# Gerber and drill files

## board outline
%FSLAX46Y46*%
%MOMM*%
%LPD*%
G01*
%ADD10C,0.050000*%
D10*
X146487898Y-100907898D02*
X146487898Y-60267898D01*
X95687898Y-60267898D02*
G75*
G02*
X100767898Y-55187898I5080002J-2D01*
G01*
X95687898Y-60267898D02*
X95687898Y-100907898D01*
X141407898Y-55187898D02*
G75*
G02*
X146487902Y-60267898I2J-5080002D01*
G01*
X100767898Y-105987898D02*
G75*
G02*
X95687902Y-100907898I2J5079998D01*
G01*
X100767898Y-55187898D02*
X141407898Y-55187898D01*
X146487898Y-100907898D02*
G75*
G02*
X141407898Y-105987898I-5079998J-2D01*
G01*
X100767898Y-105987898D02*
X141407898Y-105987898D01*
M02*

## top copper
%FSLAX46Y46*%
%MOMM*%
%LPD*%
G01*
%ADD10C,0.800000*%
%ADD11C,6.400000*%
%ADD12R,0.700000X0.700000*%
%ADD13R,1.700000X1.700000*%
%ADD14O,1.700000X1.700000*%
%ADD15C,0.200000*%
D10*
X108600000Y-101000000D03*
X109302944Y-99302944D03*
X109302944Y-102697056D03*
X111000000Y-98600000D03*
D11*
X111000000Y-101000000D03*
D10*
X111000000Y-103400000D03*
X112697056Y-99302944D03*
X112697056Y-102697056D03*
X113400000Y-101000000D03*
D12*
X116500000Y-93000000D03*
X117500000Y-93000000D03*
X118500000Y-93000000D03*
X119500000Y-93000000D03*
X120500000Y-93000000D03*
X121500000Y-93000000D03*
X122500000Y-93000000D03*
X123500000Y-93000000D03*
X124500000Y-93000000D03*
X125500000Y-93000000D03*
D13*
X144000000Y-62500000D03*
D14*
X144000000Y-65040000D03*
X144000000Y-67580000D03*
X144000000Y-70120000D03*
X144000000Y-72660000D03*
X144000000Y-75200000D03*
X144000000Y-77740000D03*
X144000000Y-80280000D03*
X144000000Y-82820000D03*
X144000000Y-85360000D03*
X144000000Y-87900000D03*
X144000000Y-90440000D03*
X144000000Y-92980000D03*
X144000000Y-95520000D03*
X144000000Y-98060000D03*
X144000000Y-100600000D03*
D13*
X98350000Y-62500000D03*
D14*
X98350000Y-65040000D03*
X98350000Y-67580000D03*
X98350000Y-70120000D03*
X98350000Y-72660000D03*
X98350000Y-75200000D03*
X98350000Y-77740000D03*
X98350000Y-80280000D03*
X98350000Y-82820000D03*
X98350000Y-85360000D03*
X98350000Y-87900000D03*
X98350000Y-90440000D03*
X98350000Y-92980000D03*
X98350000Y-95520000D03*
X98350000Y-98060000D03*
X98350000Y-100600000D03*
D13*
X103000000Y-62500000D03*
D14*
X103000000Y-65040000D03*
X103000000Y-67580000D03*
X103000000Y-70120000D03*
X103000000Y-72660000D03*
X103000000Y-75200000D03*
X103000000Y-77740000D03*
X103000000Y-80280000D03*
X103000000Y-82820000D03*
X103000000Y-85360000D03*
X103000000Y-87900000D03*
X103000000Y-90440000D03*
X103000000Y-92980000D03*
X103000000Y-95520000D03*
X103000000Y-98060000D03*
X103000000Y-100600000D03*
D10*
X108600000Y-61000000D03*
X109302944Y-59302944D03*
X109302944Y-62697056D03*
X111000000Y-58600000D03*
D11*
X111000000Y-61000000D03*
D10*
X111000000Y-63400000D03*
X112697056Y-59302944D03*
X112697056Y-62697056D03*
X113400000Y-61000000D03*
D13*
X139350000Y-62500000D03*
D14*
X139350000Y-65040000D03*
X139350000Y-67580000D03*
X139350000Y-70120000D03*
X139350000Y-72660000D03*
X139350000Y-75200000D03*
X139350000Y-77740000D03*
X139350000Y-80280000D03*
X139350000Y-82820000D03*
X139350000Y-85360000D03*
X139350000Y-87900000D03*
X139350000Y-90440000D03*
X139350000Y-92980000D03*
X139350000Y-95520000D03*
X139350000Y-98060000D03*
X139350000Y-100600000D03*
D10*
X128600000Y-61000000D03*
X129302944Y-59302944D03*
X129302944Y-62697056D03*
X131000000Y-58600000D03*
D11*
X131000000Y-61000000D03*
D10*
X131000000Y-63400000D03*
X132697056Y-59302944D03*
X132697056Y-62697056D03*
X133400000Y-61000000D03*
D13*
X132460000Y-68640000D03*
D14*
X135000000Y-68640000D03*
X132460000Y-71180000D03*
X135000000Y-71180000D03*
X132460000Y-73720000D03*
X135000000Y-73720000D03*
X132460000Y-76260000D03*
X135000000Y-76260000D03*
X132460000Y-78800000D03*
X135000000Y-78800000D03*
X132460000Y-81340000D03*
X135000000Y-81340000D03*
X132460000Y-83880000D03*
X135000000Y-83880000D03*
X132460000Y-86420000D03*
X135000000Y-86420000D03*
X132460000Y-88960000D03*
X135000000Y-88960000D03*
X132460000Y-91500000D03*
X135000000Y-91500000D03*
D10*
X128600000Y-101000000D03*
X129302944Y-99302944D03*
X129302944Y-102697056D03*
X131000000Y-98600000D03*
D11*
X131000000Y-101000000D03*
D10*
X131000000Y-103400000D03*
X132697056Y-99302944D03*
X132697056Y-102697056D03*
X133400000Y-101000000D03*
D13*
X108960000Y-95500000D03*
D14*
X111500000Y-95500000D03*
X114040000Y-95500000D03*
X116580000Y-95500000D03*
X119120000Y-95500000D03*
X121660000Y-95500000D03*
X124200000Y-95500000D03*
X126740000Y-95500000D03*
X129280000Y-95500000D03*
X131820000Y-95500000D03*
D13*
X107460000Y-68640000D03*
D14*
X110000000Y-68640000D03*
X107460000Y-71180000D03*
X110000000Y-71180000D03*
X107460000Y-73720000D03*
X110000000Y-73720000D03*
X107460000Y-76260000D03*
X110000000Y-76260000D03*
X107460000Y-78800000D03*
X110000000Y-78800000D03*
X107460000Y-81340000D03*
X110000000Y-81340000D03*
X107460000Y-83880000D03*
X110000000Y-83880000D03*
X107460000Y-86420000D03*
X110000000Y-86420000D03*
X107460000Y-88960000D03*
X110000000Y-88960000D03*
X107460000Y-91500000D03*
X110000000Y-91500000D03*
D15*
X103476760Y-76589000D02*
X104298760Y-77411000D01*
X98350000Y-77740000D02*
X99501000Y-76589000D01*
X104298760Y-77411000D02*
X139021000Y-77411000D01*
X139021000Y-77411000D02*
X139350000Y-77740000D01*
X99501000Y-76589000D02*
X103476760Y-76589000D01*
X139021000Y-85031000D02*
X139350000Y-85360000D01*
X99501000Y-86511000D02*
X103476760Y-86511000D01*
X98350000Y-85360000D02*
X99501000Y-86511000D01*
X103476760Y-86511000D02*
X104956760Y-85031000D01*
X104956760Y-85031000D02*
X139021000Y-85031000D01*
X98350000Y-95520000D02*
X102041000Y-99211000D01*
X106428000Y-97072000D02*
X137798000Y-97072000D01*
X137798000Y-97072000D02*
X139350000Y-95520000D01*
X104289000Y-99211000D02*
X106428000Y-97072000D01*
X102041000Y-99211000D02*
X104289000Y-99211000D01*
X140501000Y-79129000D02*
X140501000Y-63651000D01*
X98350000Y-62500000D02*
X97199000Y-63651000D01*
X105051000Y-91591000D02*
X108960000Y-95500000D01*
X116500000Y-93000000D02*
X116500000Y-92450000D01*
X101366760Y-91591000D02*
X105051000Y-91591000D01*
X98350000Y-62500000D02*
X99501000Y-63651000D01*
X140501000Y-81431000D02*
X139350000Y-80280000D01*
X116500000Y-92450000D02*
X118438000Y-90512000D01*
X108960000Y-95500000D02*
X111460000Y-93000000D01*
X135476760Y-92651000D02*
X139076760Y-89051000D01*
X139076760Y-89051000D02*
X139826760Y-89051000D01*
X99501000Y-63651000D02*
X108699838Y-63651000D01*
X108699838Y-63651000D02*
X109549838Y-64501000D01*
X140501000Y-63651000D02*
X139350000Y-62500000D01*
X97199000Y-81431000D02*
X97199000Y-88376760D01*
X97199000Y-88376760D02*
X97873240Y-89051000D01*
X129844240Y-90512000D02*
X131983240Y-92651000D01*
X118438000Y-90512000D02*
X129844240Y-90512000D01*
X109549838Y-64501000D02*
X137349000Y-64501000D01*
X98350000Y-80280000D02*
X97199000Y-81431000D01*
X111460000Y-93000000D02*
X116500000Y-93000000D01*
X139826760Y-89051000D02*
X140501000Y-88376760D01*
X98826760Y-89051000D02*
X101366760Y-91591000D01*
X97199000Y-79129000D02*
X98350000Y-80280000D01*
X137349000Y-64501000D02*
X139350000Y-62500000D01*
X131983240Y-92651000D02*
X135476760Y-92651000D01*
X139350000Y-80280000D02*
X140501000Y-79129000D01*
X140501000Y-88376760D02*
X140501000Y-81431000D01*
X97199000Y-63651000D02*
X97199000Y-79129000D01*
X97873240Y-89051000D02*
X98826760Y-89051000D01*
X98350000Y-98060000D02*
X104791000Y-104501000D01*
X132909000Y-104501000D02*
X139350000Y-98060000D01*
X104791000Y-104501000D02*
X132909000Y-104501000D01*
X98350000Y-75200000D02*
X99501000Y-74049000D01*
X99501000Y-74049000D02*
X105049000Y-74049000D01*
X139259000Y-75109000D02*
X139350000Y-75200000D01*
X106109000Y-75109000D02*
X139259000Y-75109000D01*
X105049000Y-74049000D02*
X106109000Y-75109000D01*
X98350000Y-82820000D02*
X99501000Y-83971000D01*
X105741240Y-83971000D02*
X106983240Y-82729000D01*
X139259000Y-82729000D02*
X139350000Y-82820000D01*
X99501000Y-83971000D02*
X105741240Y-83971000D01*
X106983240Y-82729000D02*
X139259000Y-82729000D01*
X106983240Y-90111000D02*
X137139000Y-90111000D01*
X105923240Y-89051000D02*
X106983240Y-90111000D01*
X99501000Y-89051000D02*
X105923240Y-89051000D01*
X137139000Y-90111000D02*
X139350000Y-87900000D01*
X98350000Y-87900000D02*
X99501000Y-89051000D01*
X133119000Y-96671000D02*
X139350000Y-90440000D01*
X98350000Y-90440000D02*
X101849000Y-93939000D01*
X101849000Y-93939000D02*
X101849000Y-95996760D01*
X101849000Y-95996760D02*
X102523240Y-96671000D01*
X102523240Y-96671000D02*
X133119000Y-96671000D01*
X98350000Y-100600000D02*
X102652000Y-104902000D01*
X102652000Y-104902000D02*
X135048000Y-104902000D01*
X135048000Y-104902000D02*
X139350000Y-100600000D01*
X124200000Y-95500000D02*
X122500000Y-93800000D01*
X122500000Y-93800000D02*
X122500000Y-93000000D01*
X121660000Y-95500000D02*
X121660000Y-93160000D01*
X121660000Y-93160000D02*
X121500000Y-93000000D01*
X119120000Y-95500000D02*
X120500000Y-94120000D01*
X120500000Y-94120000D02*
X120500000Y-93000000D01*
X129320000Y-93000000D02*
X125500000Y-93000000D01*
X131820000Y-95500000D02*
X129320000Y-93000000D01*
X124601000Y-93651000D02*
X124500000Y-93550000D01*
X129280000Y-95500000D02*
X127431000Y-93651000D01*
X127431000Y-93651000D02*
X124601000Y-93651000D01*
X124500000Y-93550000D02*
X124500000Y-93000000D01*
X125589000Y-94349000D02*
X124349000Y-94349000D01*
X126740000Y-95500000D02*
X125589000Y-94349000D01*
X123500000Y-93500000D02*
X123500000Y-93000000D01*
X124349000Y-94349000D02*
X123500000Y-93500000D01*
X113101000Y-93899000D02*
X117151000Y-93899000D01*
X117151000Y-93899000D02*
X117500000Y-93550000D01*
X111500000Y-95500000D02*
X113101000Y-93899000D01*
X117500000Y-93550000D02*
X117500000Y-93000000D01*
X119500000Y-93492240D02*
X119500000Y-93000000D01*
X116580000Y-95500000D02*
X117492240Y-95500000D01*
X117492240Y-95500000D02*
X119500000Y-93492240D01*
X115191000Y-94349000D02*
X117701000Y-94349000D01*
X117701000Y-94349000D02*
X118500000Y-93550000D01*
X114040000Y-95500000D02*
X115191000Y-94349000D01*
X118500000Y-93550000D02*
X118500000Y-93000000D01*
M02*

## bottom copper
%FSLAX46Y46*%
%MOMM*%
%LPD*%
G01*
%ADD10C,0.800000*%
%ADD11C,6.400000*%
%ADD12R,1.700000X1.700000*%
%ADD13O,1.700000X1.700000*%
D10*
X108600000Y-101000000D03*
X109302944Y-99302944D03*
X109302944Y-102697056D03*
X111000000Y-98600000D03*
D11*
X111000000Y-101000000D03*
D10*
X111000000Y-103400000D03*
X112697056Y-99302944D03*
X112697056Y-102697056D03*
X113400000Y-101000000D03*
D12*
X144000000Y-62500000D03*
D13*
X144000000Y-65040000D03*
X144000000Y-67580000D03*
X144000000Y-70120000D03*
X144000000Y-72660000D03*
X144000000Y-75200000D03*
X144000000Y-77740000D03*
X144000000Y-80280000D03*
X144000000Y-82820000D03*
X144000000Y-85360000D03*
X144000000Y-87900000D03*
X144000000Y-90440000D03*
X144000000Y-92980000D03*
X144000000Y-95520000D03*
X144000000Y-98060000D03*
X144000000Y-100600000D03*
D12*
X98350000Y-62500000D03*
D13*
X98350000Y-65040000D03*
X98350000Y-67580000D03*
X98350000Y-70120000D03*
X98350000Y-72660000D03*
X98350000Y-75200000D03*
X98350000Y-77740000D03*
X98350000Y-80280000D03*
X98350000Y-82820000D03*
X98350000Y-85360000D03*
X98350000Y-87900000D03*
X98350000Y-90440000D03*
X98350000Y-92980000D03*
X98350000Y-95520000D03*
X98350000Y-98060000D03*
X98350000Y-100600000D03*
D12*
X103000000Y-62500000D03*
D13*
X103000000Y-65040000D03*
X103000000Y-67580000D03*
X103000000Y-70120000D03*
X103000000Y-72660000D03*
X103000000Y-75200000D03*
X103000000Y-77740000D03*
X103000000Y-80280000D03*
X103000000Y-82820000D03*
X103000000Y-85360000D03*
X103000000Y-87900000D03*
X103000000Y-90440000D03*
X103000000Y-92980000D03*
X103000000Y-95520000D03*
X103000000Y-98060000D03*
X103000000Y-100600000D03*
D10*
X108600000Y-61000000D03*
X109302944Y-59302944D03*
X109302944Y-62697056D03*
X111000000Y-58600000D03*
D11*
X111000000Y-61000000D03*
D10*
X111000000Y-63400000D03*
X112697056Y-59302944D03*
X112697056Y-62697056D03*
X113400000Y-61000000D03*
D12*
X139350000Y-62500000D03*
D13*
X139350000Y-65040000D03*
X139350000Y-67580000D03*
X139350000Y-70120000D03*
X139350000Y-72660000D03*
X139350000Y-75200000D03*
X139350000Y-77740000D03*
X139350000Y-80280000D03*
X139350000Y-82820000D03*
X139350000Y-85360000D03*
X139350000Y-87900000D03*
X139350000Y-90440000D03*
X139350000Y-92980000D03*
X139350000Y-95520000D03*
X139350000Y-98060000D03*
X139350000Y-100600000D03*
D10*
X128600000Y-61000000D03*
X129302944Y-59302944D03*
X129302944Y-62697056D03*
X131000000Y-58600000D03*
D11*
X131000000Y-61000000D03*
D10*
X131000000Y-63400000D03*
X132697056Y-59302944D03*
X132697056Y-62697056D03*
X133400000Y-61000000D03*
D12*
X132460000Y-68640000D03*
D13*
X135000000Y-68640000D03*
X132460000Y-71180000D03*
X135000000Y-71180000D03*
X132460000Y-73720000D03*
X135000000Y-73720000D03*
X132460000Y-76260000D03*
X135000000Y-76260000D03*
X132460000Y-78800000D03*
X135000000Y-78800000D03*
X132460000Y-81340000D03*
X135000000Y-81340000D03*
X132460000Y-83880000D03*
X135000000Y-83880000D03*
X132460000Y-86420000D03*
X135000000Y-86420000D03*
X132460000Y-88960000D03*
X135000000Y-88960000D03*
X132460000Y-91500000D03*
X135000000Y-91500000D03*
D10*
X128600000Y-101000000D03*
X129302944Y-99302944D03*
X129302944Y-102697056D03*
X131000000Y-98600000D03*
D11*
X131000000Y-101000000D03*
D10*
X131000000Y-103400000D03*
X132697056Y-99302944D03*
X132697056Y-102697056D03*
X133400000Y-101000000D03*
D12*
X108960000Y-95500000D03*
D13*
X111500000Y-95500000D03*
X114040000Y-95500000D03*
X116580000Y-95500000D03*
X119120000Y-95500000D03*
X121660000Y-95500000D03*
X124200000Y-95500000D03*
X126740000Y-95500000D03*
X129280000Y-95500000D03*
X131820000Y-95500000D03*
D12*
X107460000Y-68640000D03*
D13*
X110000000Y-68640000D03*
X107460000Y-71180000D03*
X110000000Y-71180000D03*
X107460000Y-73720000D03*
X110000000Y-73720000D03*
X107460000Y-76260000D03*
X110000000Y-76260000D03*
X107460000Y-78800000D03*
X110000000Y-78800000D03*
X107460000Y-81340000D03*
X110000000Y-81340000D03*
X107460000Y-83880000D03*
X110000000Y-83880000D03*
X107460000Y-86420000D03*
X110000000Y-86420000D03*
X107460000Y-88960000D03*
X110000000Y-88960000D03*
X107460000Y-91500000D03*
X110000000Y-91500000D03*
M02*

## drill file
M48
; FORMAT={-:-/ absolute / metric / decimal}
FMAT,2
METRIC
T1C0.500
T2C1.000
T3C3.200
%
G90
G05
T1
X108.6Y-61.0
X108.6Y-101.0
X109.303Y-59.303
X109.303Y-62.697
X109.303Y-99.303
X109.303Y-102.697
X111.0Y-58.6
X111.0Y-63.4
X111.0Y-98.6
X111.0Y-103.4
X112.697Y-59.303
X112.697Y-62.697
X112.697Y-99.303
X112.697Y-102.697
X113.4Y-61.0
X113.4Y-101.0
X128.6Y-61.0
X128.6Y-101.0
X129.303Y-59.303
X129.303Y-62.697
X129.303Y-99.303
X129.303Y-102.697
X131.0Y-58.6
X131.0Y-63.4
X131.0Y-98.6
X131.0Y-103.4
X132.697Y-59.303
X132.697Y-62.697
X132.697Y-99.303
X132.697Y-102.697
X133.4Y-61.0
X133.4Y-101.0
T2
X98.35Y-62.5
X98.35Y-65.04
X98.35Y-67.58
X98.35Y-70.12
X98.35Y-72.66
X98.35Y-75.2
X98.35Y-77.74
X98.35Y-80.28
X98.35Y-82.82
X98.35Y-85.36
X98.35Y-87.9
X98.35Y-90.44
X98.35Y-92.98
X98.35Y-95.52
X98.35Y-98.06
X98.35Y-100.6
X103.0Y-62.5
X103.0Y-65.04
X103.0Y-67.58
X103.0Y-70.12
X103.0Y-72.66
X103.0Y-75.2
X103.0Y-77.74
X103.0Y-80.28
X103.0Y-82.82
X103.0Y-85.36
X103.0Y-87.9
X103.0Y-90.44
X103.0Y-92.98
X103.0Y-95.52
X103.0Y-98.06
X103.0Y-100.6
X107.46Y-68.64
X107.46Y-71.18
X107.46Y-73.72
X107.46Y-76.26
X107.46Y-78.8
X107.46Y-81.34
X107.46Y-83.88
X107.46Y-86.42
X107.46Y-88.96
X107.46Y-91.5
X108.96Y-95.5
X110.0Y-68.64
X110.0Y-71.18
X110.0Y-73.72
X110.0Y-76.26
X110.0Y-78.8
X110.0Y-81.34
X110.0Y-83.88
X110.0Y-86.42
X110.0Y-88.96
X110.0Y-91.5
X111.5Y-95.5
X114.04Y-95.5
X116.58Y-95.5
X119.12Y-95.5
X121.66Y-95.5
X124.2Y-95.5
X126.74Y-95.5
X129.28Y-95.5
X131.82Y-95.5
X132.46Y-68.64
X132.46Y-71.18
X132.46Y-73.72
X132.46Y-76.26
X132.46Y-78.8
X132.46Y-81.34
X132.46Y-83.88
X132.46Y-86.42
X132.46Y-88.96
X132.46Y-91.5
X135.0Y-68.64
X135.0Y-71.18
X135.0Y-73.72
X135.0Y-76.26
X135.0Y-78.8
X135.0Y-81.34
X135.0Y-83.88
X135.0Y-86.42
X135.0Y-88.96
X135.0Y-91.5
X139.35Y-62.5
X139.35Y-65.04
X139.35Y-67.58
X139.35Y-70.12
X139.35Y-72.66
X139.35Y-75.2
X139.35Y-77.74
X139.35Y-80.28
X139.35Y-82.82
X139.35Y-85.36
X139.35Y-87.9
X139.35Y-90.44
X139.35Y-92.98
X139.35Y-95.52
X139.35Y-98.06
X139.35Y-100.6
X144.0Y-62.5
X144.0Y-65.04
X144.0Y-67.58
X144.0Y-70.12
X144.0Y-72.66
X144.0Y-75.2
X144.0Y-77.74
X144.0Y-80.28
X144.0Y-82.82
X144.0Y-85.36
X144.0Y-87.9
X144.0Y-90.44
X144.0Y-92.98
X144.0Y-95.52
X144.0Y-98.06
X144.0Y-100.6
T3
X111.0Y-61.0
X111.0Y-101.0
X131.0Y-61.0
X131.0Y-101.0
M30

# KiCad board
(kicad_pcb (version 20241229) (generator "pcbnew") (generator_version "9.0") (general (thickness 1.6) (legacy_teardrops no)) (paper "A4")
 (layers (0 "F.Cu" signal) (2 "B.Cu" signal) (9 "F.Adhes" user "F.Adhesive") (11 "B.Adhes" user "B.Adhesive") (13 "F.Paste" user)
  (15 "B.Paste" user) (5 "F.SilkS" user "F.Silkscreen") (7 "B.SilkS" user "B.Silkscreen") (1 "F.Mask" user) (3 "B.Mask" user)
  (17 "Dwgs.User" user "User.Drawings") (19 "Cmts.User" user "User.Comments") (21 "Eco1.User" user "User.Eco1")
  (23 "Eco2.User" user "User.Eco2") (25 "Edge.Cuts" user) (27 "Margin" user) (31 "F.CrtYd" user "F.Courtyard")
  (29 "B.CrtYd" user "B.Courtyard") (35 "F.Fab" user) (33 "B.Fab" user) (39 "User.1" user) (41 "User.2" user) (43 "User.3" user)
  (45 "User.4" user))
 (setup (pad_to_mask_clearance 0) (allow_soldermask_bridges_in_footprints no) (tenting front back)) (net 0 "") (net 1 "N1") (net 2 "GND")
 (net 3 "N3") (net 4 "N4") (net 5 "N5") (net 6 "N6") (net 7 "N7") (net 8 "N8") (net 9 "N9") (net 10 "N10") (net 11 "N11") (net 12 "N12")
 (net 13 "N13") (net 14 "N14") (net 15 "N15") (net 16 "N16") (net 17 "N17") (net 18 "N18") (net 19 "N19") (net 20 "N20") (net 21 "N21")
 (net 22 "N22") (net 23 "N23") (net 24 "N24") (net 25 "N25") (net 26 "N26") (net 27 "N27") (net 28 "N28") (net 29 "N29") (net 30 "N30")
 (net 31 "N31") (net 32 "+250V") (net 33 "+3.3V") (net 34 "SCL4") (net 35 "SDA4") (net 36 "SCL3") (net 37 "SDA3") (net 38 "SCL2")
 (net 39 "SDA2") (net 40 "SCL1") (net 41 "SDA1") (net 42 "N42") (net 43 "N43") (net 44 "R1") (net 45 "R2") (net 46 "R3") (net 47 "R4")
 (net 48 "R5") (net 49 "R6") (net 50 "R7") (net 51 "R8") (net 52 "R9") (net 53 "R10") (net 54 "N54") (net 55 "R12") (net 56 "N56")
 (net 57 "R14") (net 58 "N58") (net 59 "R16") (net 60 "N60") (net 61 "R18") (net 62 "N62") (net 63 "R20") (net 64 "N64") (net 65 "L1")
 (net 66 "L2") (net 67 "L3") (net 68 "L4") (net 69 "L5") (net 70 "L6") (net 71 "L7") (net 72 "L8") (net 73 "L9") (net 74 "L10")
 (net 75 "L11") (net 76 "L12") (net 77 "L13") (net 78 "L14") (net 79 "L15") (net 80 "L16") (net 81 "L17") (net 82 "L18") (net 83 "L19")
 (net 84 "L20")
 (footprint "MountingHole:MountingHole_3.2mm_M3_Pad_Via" (layer "F.Cu") (at 111 101)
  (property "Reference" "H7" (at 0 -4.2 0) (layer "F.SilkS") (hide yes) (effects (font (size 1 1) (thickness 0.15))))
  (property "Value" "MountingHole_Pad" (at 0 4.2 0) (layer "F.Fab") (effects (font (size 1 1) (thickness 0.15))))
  (pad "1" thru_hole circle (at -2.4 0) (size 0.8 0.8) (drill 0.5) (layers "*.Cu" "*.Mask") (remove_unused_layers no) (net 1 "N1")
   (zone_connect 2))
  (pad "1" thru_hole circle (at -1.697056 -1.697056) (size 0.8 0.8) (drill 0.5) (layers "*.Cu" "*.Mask") (remove_unused_layers no)
   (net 1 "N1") (zone_connect 2))
  (pad "1" thru_hole circle (at -1.697056 1.697056) (size 0.8 0.8) (drill 0.5) (layers "*.Cu" "*.Mask") (remove_unused_layers no)
   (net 1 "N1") (zone_connect 2))
  (pad "1" thru_hole circle (at 0 -2.4) (size 0.8 0.8) (drill 0.5) (layers "*.Cu" "*.Mask") (remove_unused_layers no) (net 1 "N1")
   (zone_connect 2))
  (pad "1" thru_hole circle (at 0 0) (size 6.4 6.4) (drill 3.2) (layers "*.Cu" "*.Mask") (remove_unused_layers no) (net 1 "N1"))
  (pad "1" thru_hole circle (at 0 2.4) (size 0.8 0.8) (drill 0.5) (layers "*.Cu" "*.Mask") (remove_unused_layers no) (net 1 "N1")
   (zone_connect 2))
  (pad "1" thru_hole circle (at 1.697056 -1.697056) (size 0.8 0.8) (drill 0.5) (layers "*.Cu" "*.Mask") (remove_unused_layers no)
   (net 1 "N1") (zone_connect 2))
  (pad "1" thru_hole circle (at 1.697056 1.697056) (size 0.8 0.8) (drill 0.5) (layers "*.Cu" "*.Mask") (remove_unused_layers no)
   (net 1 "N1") (zone_connect 2))
  (pad "1" thru_hole circle (at 2.4 0) (size 0.8 0.8) (drill 0.5) (layers "*.Cu" "*.Mask") (remove_unused_layers no) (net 1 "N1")
   (zone_connect 2)))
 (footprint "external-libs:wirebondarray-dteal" (layer "F.Cu") (at 116.5 93)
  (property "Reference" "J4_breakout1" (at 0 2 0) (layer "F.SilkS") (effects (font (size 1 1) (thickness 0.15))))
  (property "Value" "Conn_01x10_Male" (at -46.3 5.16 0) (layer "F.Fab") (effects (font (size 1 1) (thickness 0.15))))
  (pad "1" smd rect (at 0 0) (size 0.7 0.7) (layers "F.Cu" "F.Mask" "F.Paste") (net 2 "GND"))
  (pad "2" smd rect (at 1 0) (size 0.7 0.7) (layers "F.Cu" "F.Mask" "F.Paste") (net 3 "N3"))
  (pad "3" smd rect (at 2 0) (size 0.7 0.7) (layers "F.Cu" "F.Mask" "F.Paste") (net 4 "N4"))
  (pad "4" smd rect (at 3 0) (size 0.7 0.7) (layers "F.Cu" "F.Mask" "F.Paste") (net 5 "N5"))
  (pad "5" smd rect (at 4 0) (size 0.7 0.7) (layers "F.Cu" "F.Mask" "F.Paste") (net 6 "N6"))
  (pad "6" smd rect (at 5 0) (size 0.7 0.7) (layers "F.Cu" "F.Mask" "F.Paste") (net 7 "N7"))
  (pad "7" smd rect (at 6 0) (size 0.7 0.7) (layers "F.Cu" "F.Mask" "F.Paste") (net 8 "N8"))
  (pad "8" smd rect (at 7 0) (size 0.7 0.7) (layers "F.Cu" "F.Mask" "F.Paste") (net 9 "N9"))
  (pad "9" smd rect (at 8 0) (size 0.7 0.7) (layers "F.Cu" "F.Mask" "F.Paste") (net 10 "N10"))
  (pad "10" smd rect (at 9 0) (size 0.7 0.7) (layers "F.Cu" "F.Mask" "F.Paste") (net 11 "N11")))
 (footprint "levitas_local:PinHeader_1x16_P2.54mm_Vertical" (layer "F.Cu") (at 144 62.5)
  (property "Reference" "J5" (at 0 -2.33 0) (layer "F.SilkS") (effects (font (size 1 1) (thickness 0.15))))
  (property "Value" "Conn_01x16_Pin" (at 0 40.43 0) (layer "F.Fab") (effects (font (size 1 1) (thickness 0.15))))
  (pad "1" thru_hole rect (at 0 0) (size 1.7 1.7) (drill 1) (layers "*.Cu" "*.Mask") (remove_unused_layers no) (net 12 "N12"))
  (pad "2" thru_hole oval (at 0 2.54) (size 1.7 1.7) (drill 1) (layers "*.Cu" "*.Mask") (remove_unused_layers no) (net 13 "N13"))
  (pad "3" thru_hole oval (at 0 5.08) (size 1.7 1.7) (drill 1) (layers "*.Cu" "*.Mask") (remove_unused_layers no) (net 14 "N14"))
  (pad "4" thru_hole oval (at 0 7.62) (size 1.7 1.7) (drill 1) (layers "*.Cu" "*.Mask") (remove_unused_layers no) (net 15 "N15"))
  (pad "5" thru_hole oval (at 0 10.16) (size 1.7 1.7) (drill 1) (layers "*.Cu" "*.Mask") (remove_unused_layers no) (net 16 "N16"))
  (pad "6" thru_hole oval (at 0 12.7) (size 1.7 1.7) (drill 1) (layers "*.Cu" "*.Mask") (remove_unused_layers no) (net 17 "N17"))
  (pad "7" thru_hole oval (at 0 15.24) (size 1.7 1.7) (drill 1) (layers "*.Cu" "*.Mask") (remove_unused_layers no) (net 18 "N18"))
  (pad "8" thru_hole oval (at 0 17.78) (size 1.7 1.7) (drill 1) (layers "*.Cu" "*.Mask") (remove_unused_layers no) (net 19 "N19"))
  (pad "9" thru_hole oval (at 0 20.32) (size 1.7 1.7) (drill 1) (layers "*.Cu" "*.Mask") (remove_unused_layers no) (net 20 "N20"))
  (pad "10" thru_hole oval (at 0 22.86) (size 1.7 1.7) (drill 1) (layers "*.Cu" "*.Mask") (remove_unused_layers no) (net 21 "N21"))
  (pad "11" thru_hole oval (at 0 25.4) (size 1.7 1.7) (drill 1) (layers "*.Cu" "*.Mask") (remove_unused_layers no) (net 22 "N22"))
  (pad "12" thru_hole oval (at 0 27.94) (size 1.7 1.7) (drill 1) (layers "*.Cu" "*.Mask") (remove_unused_layers no) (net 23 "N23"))
  (pad "13" thru_hole oval (at 0 30.48) (size 1.7 1.7) (drill 1) (layers "*.Cu" "*.Mask") (remove_unused_layers no) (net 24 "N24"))
  (pad "14" thru_hole oval (at 0 33.02) (size 1.7 1.7) (drill 1) (layers "*.Cu" "*.Mask") (remove_unused_layers no) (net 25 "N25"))
  (pad "15" thru_hole oval (at 0 35.56) (size 1.7 1.7) (drill 1) (layers "*.Cu" "*.Mask") (remove_unused_layers no) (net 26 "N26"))
  (pad "16" thru_hole oval (at 0 38.1) (size 1.7 1.7) (drill 1) (layers "*.Cu" "*.Mask") (remove_unused_layers no) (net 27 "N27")))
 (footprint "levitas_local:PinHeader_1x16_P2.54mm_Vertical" (layer "F.Cu") (at 98.35 62.5)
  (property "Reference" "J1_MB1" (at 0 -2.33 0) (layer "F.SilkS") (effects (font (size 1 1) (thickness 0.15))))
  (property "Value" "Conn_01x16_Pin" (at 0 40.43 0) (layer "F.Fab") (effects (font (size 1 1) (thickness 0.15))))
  (pad "1" thru_hole rect (at 0 0) (size 1.7 1.7) (drill 1) (layers "*.Cu" "*.Mask") (remove_unused_layers no) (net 2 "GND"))
  (pad "2" thru_hole oval (at 0 2.54) (size 1.7 1.7) (drill 1) (layers "*.Cu" "*.Mask") (remove_unused_layers no) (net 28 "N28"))
  (pad "3" thru_hole oval (at 0 5.08) (size 1.7 1.7) (drill 1) (layers "*.Cu" "*.Mask") (remove_unused_layers no) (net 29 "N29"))
  (pad "4" thru_hole oval (at 0 7.62) (size 1.7 1.7) (drill 1) (layers "*.Cu" "*.Mask") (remove_unused_layers no) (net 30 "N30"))
  (pad "5" thru_hole oval (at 0 10.16) (size 1.7 1.7) (drill 1) (layers "*.Cu" "*.Mask") (remove_unused_layers no) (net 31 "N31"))
  (pad "6" thru_hole oval (at 0 12.7) (size 1.7 1.7) (drill 1) (layers "*.Cu" "*.Mask") (remove_unused_layers no) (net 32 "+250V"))
  (pad "7" thru_hole oval (at 0 15.24) (size 1.7 1.7) (drill 1) (layers "*.Cu" "*.Mask") (remove_unused_layers no) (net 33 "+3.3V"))
  (pad "8" thru_hole oval (at 0 17.78) (size 1.7 1.7) (drill 1) (layers "*.Cu" "*.Mask") (remove_unused_layers no) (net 2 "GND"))
  (pad "9" thru_hole oval (at 0 20.32) (size 1.7 1.7) (drill 1) (layers "*.Cu" "*.Mask") (remove_unused_layers no) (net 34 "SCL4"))
  (pad "10" thru_hole oval (at 0 22.86) (size 1.7 1.7) (drill 1) (layers "*.Cu" "*.Mask") (remove_unused_layers no) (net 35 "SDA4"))
  (pad "11" thru_hole oval (at 0 25.4) (size 1.7 1.7) (drill 1) (layers "*.Cu" "*.Mask") (remove_unused_layers no) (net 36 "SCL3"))
  (pad "12" thru_hole oval (at 0 27.94) (size 1.7 1.7) (drill 1) (layers "*.Cu" "*.Mask") (remove_unused_layers no) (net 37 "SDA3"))
  (pad "13" thru_hole oval (at 0 30.48) (size 1.7 1.7) (drill 1) (layers "*.Cu" "*.Mask") (remove_unused_layers no) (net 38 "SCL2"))
  (pad "14" thru_hole oval (at 0 33.02) (size 1.7 1.7) (drill 1) (layers "*.Cu" "*.Mask") (remove_unused_layers no) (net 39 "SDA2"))
  (pad "15" thru_hole oval (at 0 35.56) (size 1.7 1.7) (drill 1) (layers "*.Cu" "*.Mask") (remove_unused_layers no) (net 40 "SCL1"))
  (pad "16" thru_hole oval (at 0 38.1) (size 1.7 1.7) (drill 1) (layers "*.Cu" "*.Mask") (remove_unused_layers no) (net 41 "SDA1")))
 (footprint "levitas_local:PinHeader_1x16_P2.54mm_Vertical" (layer "F.Cu") (at 103 62.5)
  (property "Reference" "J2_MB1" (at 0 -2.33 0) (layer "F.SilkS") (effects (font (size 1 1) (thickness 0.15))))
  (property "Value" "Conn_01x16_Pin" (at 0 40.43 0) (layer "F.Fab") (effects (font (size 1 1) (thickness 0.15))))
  (pad "1" thru_hole rect (at 0 0) (size 1.7 1.7) (drill 1) (layers "*.Cu" "*.Mask") (remove_unused_layers no) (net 12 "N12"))
  (pad "2" thru_hole oval (at 0 2.54) (size 1.7 1.7) (drill 1) (layers "*.Cu" "*.Mask") (remove_unused_layers no) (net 13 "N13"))
  (pad "3" thru_hole oval (at 0 5.08) (size 1.7 1.7) (drill 1) (layers "*.Cu" "*.Mask") (remove_unused_layers no) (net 14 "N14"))
  (pad "4" thru_hole oval (at 0 7.62) (size 1.7 1.7) (drill 1) (layers "*.Cu" "*.Mask") (remove_unused_layers no) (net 15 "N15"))
  (pad "5" thru_hole oval (at 0 10.16) (size 1.7 1.7) (drill 1) (layers "*.Cu" "*.Mask") (remove_unused_layers no) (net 16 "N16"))
  (pad "6" thru_hole oval (at 0 12.7) (size 1.7 1.7) (drill 1) (layers "*.Cu" "*.Mask") (remove_unused_layers no) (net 17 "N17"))
  (pad "7" thru_hole oval (at 0 15.24) (size 1.7 1.7) (drill 1) (layers "*.Cu" "*.Mask") (remove_unused_layers no) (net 18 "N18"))
  (pad "8" thru_hole oval (at 0 17.78) (size 1.7 1.7) (drill 1) (layers "*.Cu" "*.Mask") (remove_unused_layers no) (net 19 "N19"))
  (pad "9" thru_hole oval (at 0 20.32) (size 1.7 1.7) (drill 1) (layers "*.Cu" "*.Mask") (remove_unused_layers no) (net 20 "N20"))
  (pad "10" thru_hole oval (at 0 22.86) (size 1.7 1.7) (drill 1) (layers "*.Cu" "*.Mask") (remove_unused_layers no) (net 21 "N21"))
  (pad "11" thru_hole oval (at 0 25.4) (size 1.7 1.7) (drill 1) (layers "*.Cu" "*.Mask") (remove_unused_layers no) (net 22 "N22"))
  (pad "12" thru_hole oval (at 0 27.94) (size 1.7 1.7) (drill 1) (layers "*.Cu" "*.Mask") (remove_unused_layers no) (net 23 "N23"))
  (pad "13" thru_hole oval (at 0 30.48) (size 1.7 1.7) (drill 1) (layers "*.Cu" "*.Mask") (remove_unused_layers no) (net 24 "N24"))
  (pad "14" thru_hole oval (at 0 33.02) (size 1.7 1.7) (drill 1) (layers "*.Cu" "*.Mask") (remove_unused_layers no) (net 25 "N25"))
  (pad "15" thru_hole oval (at 0 35.56) (size 1.7 1.7) (drill 1) (layers "*.Cu" "*.Mask") (remove_unused_layers no) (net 26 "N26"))
  (pad "16" thru_hole oval (at 0 38.1) (size 1.7 1.7) (drill 1) (layers "*.Cu" "*.Mask") (remove_unused_layers no) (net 27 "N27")))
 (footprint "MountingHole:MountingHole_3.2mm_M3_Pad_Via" (layer "F.Cu") (at 111 61)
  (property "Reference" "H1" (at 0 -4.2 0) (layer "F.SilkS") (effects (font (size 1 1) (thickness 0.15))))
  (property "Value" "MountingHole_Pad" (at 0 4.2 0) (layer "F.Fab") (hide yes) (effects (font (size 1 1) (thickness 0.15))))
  (pad "1" thru_hole circle (at -2.4 0) (size 0.8 0.8) (drill 0.5) (layers "*.Cu" "*.Mask") (remove_unused_layers no) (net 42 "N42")
   (zone_connect 2))
  (pad "1" thru_hole circle (at -1.697056 -1.697056) (size 0.8 0.8) (drill 0.5) (layers "*.Cu" "*.Mask") (remove_unused_layers no)
   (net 42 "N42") (zone_connect 2))
  (pad "1" thru_hole circle (at -1.697056 1.697056) (size 0.8 0.8) (drill 0.5) (layers "*.Cu" "*.Mask") (remove_unused_layers no)
   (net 42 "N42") (zone_connect 2))
  (pad "1" thru_hole circle (at 0 -2.4) (size 0.8 0.8) (drill 0.5) (layers "*.Cu" "*.Mask") (remove_unused_layers no) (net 42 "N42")
   (zone_connect 2))
  (pad "1" thru_hole circle (at 0 0) (size 6.4 6.4) (drill 3.2) (layers "*.Cu" "*.Mask") (remove_unused_layers no) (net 42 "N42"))
  (pad "1" thru_hole circle (at 0 2.4) (size 0.8 0.8) (drill 0.5) (layers "*.Cu" "*.Mask") (remove_unused_layers no) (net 42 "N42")
   (zone_connect 2))
  (pad "1" thru_hole circle (at 1.697056 -1.697056) (size 0.8 0.8) (drill 0.5) (layers "*.Cu" "*.Mask") (remove_unused_layers no)
   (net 42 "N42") (zone_connect 2))
  (pad "1" thru_hole circle (at 1.697056 1.697056) (size 0.8 0.8) (drill 0.5) (layers "*.Cu" "*.Mask") (remove_unused_layers no)
   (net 42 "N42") (zone_connect 2))
  (pad "1" thru_hole circle (at 2.4 0) (size 0.8 0.8) (drill 0.5) (layers "*.Cu" "*.Mask") (remove_unused_layers no) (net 42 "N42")
   (zone_connect 2)))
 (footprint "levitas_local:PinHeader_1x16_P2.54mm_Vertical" (layer "F.Cu") (at 139.35 62.5)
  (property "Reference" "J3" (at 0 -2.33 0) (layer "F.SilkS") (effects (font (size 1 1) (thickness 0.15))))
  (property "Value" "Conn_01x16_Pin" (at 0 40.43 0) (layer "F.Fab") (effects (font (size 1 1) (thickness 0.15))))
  (pad "1" thru_hole rect (at 0 0) (size 1.7 1.7) (drill 1) (layers "*.Cu" "*.Mask") (remove_unused_layers no) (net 2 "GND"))
  (pad "2" thru_hole oval (at 0 2.54) (size 1.7 1.7) (drill 1) (layers "*.Cu" "*.Mask") (remove_unused_layers no) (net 28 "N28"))
  (pad "3" thru_hole oval (at 0 5.08) (size 1.7 1.7) (drill 1) (layers "*.Cu" "*.Mask") (remove_unused_layers no) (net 29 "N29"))
  (pad "4" thru_hole oval (at 0 7.62) (size 1.7 1.7) (drill 1) (layers "*.Cu" "*.Mask") (remove_unused_layers no) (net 30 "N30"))
  (pad "5" thru_hole oval (at 0 10.16) (size 1.7 1.7) (drill 1) (layers "*.Cu" "*.Mask") (remove_unused_layers no) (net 31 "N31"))
  (pad "6" thru_hole oval (at 0 12.7) (size 1.7 1.7) (drill 1) (layers "*.Cu" "*.Mask") (remove_unused_layers no) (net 32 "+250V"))
  (pad "7" thru_hole oval (at 0 15.24) (size 1.7 1.7) (drill 1) (layers "*.Cu" "*.Mask") (remove_unused_layers no) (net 33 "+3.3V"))
  (pad "8" thru_hole oval (at 0 17.78) (size 1.7 1.7) (drill 1) (layers "*.Cu" "*.Mask") (remove_unused_layers no) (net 2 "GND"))
  (pad "9" thru_hole oval (at 0 20.32) (size 1.7 1.7) (drill 1) (layers "*.Cu" "*.Mask") (remove_unused_layers no) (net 34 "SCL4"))
  (pad "10" thru_hole oval (at 0 22.86) (size 1.7 1.7) (drill 1) (layers "*.Cu" "*.Mask") (remove_unused_layers no) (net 35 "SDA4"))
  (pad "11" thru_hole oval (at 0 25.4) (size 1.7 1.7) (drill 1) (layers "*.Cu" "*.Mask") (remove_unused_layers no) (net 36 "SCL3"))
  (pad "12" thru_hole oval (at 0 27.94) (size 1.7 1.7) (drill 1) (layers "*.Cu" "*.Mask") (remove_unused_layers no) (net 37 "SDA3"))
  (pad "13" thru_hole oval (at 0 30.48) (size 1.7 1.7) (drill 1) (layers "*.Cu" "*.Mask") (remove_unused_layers no) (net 38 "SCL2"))
  (pad "14" thru_hole oval (at 0 33.02) (size 1.7 1.7) (drill 1) (layers "*.Cu" "*.Mask") (remove_unused_layers no) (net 39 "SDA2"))
  (pad "15" thru_hole oval (at 0 35.56) (size 1.7 1.7) (drill 1) (layers "*.Cu" "*.Mask") (remove_unused_layers no) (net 40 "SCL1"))
  (pad "16" thru_hole oval (at 0 38.1) (size 1.7 1.7) (drill 1) (layers "*.Cu" "*.Mask") (remove_unused_layers no) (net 41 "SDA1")))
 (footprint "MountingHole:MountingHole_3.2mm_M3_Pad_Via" (layer "F.Cu") (at 131 61)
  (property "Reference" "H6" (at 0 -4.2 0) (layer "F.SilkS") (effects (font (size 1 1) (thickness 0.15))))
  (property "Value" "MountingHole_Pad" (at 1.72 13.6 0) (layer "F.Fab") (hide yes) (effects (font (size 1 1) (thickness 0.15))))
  (pad "1" thru_hole circle (at -2.4 0) (size 0.8 0.8) (drill 0.5) (layers "*.Cu" "*.Mask") (remove_unused_layers no) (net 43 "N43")
   (zone_connect 2))
  (pad "1" thru_hole circle (at -1.697056 -1.697056) (size 0.8 0.8) (drill 0.5) (layers "*.Cu" "*.Mask") (remove_unused_layers no)
   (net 43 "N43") (zone_connect 2))
  (pad "1" thru_hole circle (at -1.697056 1.697056) (size 0.8 0.8) (drill 0.5) (layers "*.Cu" "*.Mask") (remove_unused_layers no)
   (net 43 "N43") (zone_connect 2))
  (pad "1" thru_hole circle (at 0 -2.4) (size 0.8 0.8) (drill 0.5) (layers "*.Cu" "*.Mask") (remove_unused_layers no) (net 43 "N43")
   (zone_connect 2))
  (pad "1" thru_hole circle (at 0 0) (size 6.4 6.4) (drill 3.2) (layers "*.Cu" "*.Mask") (remove_unused_layers no) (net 43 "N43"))
  (pad "1" thru_hole circle (at 0 2.4) (size 0.8 0.8) (drill 0.5) (layers "*.Cu" "*.Mask") (remove_unused_layers no) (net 43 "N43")
   (zone_connect 2))
  (pad "1" thru_hole circle (at 1.697056 -1.697056) (size 0.8 0.8) (drill 0.5) (layers "*.Cu" "*.Mask") (remove_unused_layers no)
   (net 43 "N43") (zone_connect 2))
  (pad "1" thru_hole circle (at 1.697056 1.697056) (size 0.8 0.8) (drill 0.5) (layers "*.Cu" "*.Mask") (remove_unused_layers no)
   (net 43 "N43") (zone_connect 2))
  (pad "1" thru_hole circle (at 2.4 0) (size 0.8 0.8) (drill 0.5) (layers "*.Cu" "*.Mask") (remove_unused_layers no) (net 43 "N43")
   (zone_connect 2)))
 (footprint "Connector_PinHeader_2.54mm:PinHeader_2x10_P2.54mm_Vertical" (layer "F.Cu") (at 132.46 68.64)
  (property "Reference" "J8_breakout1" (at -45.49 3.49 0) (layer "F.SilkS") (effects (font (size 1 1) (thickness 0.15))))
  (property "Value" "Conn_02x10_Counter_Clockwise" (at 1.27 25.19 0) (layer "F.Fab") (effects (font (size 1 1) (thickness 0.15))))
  (pad "1" thru_hole rect (at 0 0) (size 1.7 1.7) (drill 1) (layers "*.Cu" "*.Mask") (remove_unused_layers no) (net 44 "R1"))
  (pad "2" thru_hole oval (at 2.54 0) (size 1.7 1.7) (drill 1) (layers "*.Cu" "*.Mask") (remove_unused_layers no) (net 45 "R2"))
  (pad "3" thru_hole oval (at 0 2.54) (size 1.7 1.7) (drill 1) (layers "*.Cu" "*.Mask") (remove_unused_layers no) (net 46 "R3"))
  (pad "4" thru_hole oval (at 2.54 2.54) (size 1.7 1.7) (drill 1) (layers "*.Cu" "*.Mask") (remove_unused_layers no) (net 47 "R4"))
  (pad "5" thru_hole oval (at 0 5.08) (size 1.7 1.7) (drill 1) (layers "*.Cu" "*.Mask") (remove_unused_layers no) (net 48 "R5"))
  (pad "6" thru_hole oval (at 2.54 5.08) (size 1.7 1.7) (drill 1) (layers "*.Cu" "*.Mask") (remove_unused_layers no) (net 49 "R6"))
  (pad "7" thru_hole oval (at 0 7.62) (size 1.7 1.7) (drill 1) (layers "*.Cu" "*.Mask") (remove_unused_layers no) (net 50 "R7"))
  (pad "8" thru_hole oval (at 2.54 7.62) (size 1.7 1.7) (drill 1) (layers "*.Cu" "*.Mask") (remove_unused_layers no) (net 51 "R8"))
  (pad "9" thru_hole oval (at 0 10.16) (size 1.7 1.7) (drill 1) (layers "*.Cu" "*.Mask") (remove_unused_layers no) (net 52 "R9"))
  (pad "10" thru_hole oval (at 2.54 10.16) (size 1.7 1.7) (drill 1) (layers "*.Cu" "*.Mask") (remove_unused_layers no) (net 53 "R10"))
  (pad "11" thru_hole oval (at 0 12.7) (size 1.7 1.7) (drill 1) (layers "*.Cu" "*.Mask") (remove_unused_layers no) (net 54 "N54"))
  (pad "12" thru_hole oval (at 2.54 12.7) (size 1.7 1.7) (drill 1) (layers "*.Cu" "*.Mask") (remove_unused_layers no) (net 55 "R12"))
  (pad "13" thru_hole oval (at 0 15.24) (size 1.7 1.7) (drill 1) (layers "*.Cu" "*.Mask") (remove_unused_layers no) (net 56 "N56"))
  (pad "14" thru_hole oval (at 2.54 15.24) (size 1.7 1.7) (drill 1) (layers "*.Cu" "*.Mask") (remove_unused_layers no) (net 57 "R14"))
  (pad "15" thru_hole oval (at 0 17.78) (size 1.7 1.7) (drill 1) (layers "*.Cu" "*.Mask") (remove_unused_layers no) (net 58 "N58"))
  (pad "16" thru_hole oval (at 2.54 17.78) (size 1.7 1.7) (drill 1) (layers "*.Cu" "*.Mask") (remove_unused_layers no) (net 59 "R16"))
  (pad "17" thru_hole oval (at 0 20.32) (size 1.7 1.7) (drill 1) (layers "*.Cu" "*.Mask") (remove_unused_layers no) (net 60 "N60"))
  (pad "18" thru_hole oval (at 2.54 20.32) (size 1.7 1.7) (drill 1) (layers "*.Cu" "*.Mask") (remove_unused_layers no) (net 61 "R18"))
  (pad "19" thru_hole oval (at 0 22.86) (size 1.7 1.7) (drill 1) (layers "*.Cu" "*.Mask") (remove_unused_layers no) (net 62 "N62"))
  (pad "20" thru_hole oval (at 2.54 22.86) (size 1.7 1.7) (drill 1) (layers "*.Cu" "*.Mask") (remove_unused_layers no) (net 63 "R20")))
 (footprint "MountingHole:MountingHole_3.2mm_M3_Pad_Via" (layer "F.Cu") (at 131 101)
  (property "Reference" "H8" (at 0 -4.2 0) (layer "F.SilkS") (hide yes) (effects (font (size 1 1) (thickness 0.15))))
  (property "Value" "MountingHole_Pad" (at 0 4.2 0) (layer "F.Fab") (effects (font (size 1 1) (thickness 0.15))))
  (pad "1" thru_hole circle (at -2.4 0) (size 0.8 0.8) (drill 0.5) (layers "*.Cu" "*.Mask") (remove_unused_layers no) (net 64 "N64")
   (zone_connect 2))
  (pad "1" thru_hole circle (at -1.697056 -1.697056) (size 0.8 0.8) (drill 0.5) (layers "*.Cu" "*.Mask") (remove_unused_layers no)
   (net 64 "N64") (zone_connect 2))
  (pad "1" thru_hole circle (at -1.697056 1.697056) (size 0.8 0.8) (drill 0.5) (layers "*.Cu" "*.Mask") (remove_unused_layers no)
   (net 64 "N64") (zone_connect 2))
  (pad "1" thru_hole circle (at 0 -2.4) (size 0.8 0.8) (drill 0.5) (layers "*.Cu" "*.Mask") (remove_unused_layers no) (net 64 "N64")
   (zone_connect 2))
  (pad "1" thru_hole circle (at 0 0) (size 6.4 6.4) (drill 3.2) (layers "*.Cu" "*.Mask") (remove_unused_layers no) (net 64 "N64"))
  (pad "1" thru_hole circle (at 0 2.4) (size 0.8 0.8) (drill 0.5) (layers "*.Cu" "*.Mask") (remove_unused_layers no) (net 64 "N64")
   (zone_connect 2))
  (pad "1" thru_hole circle (at 1.697056 -1.697056) (size 0.8 0.8) (drill 0.5) (layers "*.Cu" "*.Mask") (remove_unused_layers no)
   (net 64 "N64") (zone_connect 2))
  (pad "1" thru_hole circle (at 1.697056 1.697056) (size 0.8 0.8) (drill 0.5) (layers "*.Cu" "*.Mask") (remove_unused_layers no)
   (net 64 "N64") (zone_connect 2))
  (pad "1" thru_hole circle (at 2.4 0) (size 0.8 0.8) (drill 0.5) (layers "*.Cu" "*.Mask") (remove_unused_layers no) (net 64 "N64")
   (zone_connect 2)))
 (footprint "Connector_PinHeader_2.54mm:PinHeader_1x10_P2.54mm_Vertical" (layer "F.Cu") (at 108.96 95.5 90)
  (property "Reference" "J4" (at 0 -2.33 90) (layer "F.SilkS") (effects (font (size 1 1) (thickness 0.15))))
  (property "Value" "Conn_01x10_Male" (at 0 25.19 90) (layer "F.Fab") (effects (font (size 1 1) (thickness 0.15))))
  (pad "1" thru_hole rect (at 0 0 90) (size 1.7 1.7) (drill 1) (layers "*.Cu" "*.Mask") (remove_unused_layers no) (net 2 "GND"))
  (pad "2" thru_hole oval (at 0 2.54 90) (size 1.7 1.7) (drill 1) (layers "*.Cu" "*.Mask") (remove_unused_layers no) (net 3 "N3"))
  (pad "3" thru_hole oval (at 0 5.08 90) (size 1.7 1.7) (drill 1) (layers "*.Cu" "*.Mask") (remove_unused_layers no) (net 4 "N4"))
  (pad "4" thru_hole oval (at 0 7.62 90) (size 1.7 1.7) (drill 1) (layers "*.Cu" "*.Mask") (remove_unused_layers no) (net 5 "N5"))
  (pad "5" thru_hole oval (at 0 10.16 90) (size 1.7 1.7) (drill 1) (layers "*.Cu" "*.Mask") (remove_unused_layers no) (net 6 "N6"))
  (pad "6" thru_hole oval (at 0 12.7 90) (size 1.7 1.7) (drill 1) (layers "*.Cu" "*.Mask") (remove_unused_layers no) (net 7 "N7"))
  (pad "7" thru_hole oval (at 0 15.24 90) (size 1.7 1.7) (drill 1) (layers "*.Cu" "*.Mask") (remove_unused_layers no) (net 8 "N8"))
  (pad "8" thru_hole oval (at 0 17.78 90) (size 1.7 1.7) (drill 1) (layers "*.Cu" "*.Mask") (remove_unused_layers no) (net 9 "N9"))
  (pad "9" thru_hole oval (at 0 20.32 90) (size 1.7 1.7) (drill 1) (layers "*.Cu" "*.Mask") (remove_unused_layers no) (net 10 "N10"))
  (pad "10" thru_hole oval (at 0 22.86 90) (size 1.7 1.7) (drill 1) (layers "*.Cu" "*.Mask") (remove_unused_layers no) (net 11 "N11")))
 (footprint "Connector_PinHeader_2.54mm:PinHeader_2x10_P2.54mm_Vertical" (layer "F.Cu") (at 107.46 68.64)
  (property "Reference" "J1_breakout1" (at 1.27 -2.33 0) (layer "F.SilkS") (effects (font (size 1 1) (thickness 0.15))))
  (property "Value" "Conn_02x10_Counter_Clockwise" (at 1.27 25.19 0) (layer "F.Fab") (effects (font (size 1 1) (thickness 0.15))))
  (pad "1" thru_hole rect (at 0 0) (size 1.7 1.7) (drill 1) (layers "*.Cu" "*.Mask") (remove_unused_layers no) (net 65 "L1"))
  (pad "2" thru_hole oval (at 2.54 0) (size 1.7 1.7) (drill 1) (layers "*.Cu" "*.Mask") (remove_unused_layers no) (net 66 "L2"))
  (pad "3" thru_hole oval (at 0 2.54) (size 1.7 1.7) (drill 1) (layers "*.Cu" "*.Mask") (remove_unused_layers no) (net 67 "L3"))
  (pad "4" thru_hole oval (at 2.54 2.54) (size 1.7 1.7) (drill 1) (layers "*.Cu" "*.Mask") (remove_unused_layers no) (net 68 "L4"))
  (pad "5" thru_hole oval (at 0 5.08) (size 1.7 1.7) (drill 1) (layers "*.Cu" "*.Mask") (remove_unused_layers no) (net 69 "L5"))
  (pad "6" thru_hole oval (at 2.54 5.08) (size 1.7 1.7) (drill 1) (layers "*.Cu" "*.Mask") (remove_unused_layers no) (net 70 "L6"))
  (pad "7" thru_hole oval (at 0 7.62) (size 1.7 1.7) (drill 1) (layers "*.Cu" "*.Mask") (remove_unused_layers no) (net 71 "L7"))
  (pad "8" thru_hole oval (at 2.54 7.62) (size 1.7 1.7) (drill 1) (layers "*.Cu" "*.Mask") (remove_unused_layers no) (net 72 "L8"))
  (pad "9" thru_hole oval (at 0 10.16) (size 1.7 1.7) (drill 1) (layers "*.Cu" "*.Mask") (remove_unused_layers no) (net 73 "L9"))
  (pad "10" thru_hole oval (at 2.54 10.16) (size 1.7 1.7) (drill 1) (layers "*.Cu" "*.Mask") (remove_unused_layers no) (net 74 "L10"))
  (pad "11" thru_hole oval (at 0 12.7) (size 1.7 1.7) (drill 1) (layers "*.Cu" "*.Mask") (remove_unused_layers no) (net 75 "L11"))
  (pad "12" thru_hole oval (at 2.54 12.7) (size 1.7 1.7) (drill 1) (layers "*.Cu" "*.Mask") (remove_unused_layers no) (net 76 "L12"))
  (pad "13" thru_hole oval (at 0 15.24) (size 1.7 1.7) (drill 1) (layers "*.Cu" "*.Mask") (remove_unused_layers no) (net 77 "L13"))
  (pad "14" thru_hole oval (at 2.54 15.24) (size 1.7 1.7) (drill 1) (layers "*.Cu" "*.Mask") (remove_unused_layers no) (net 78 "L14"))
  (pad "15" thru_hole oval (at 0 17.78) (size 1.7 1.7) (drill 1) (layers "*.Cu" "*.Mask") (remove_unused_layers no) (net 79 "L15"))
  (pad "16" thru_hole oval (at 2.54 17.78) (size 1.7 1.7) (drill 1) (layers "*.Cu" "*.Mask") (remove_unused_layers no) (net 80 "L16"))
  (pad "17" thru_hole oval (at 0 20.32) (size 1.7 1.7) (drill 1) (layers "*.Cu" "*.Mask") (remove_unused_layers no) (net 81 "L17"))
  (pad "18" thru_hole oval (at 2.54 20.32) (size 1.7 1.7) (drill 1) (layers "*.Cu" "*.Mask") (remove_unused_layers no) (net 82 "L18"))
  (pad "19" thru_hole oval (at 0 22.86) (size 1.7 1.7) (drill 1) (layers "*.Cu" "*.Mask") (remove_unused_layers no) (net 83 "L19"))
  (pad "20" thru_hole oval (at 2.54 22.86) (size 1.7 1.7) (drill 1) (layers "*.Cu" "*.Mask") (remove_unused_layers no) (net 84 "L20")))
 (gr_line (start 146.487898 100.907898) (end 146.487898 60.267898) (stroke (width 0.05) (type default)) (layer "Edge.Cuts"))
 (gr_arc (start 95.687898 60.267898) (mid 97.175796 56.675796) (end 100.767898 55.187898) (stroke (width 0.05) (type default))
  (layer "Edge.Cuts"))
 (gr_line (start 95.687898 60.267898) (end 95.687898 100.907898) (stroke (width 0.05) (type default)) (layer "Edge.Cuts"))
 (gr_arc (start 141.407898 55.187898) (mid 145 56.675796) (end 146.487898 60.267898) (stroke (width 0.05) (type default))
  (layer "Edge.Cuts"))
 (gr_arc (start 100.767898 105.987898) (mid 97.175796 104.5) (end 95.687898 100.907898) (stroke (width 0.05) (type default))
  (layer "Edge.Cuts"))
 (gr_line (start 100.767898 55.187898) (end 141.407898 55.187898) (stroke (width 0.05) (type default)) (layer "Edge.Cuts"))
 (gr_arc (start 146.487898 100.907898) (mid 145 104.5) (end 141.407898 105.987898) (stroke (width 0.05) (type default)) (layer "Edge.Cuts"))
 (gr_line (start 100.767898 105.987898) (end 141.407898 105.987898) (stroke (width 0.05) (type default)) (layer "Edge.Cuts"))
 (segment (start 103.47676 76.589) (end 104.29876 77.411) (width 0.2) (layer "F.Cu") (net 33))
 (segment (start 98.35 77.74) (end 99.501 76.589) (width 0.2) (layer "F.Cu") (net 33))
 (segment (start 104.29876 77.411) (end 139.021 77.411) (width 0.2) (layer "F.Cu") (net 33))
 (segment (start 139.021 77.411) (end 139.35 77.74) (width 0.2) (layer "F.Cu") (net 33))
 (segment (start 99.501 76.589) (end 103.47676 76.589) (width 0.2) (layer "F.Cu") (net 33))
 (segment (start 139.021 85.031) (end 139.35 85.36) (width 0.2) (layer "F.Cu") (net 35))
 (segment (start 99.501 86.511) (end 103.47676 86.511) (width 0.2) (layer "F.Cu") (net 35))
 (segment (start 98.35 85.36) (end 99.501 86.511) (width 0.2) (layer "F.Cu") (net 35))
 (segment (start 103.47676 86.511) (end 104.95676 85.031) (width 0.2) (layer "F.Cu") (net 35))
 (segment (start 104.95676 85.031) (end 139.021 85.031) (width 0.2) (layer "F.Cu") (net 35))
 (segment (start 98.35 95.52) (end 102.041 99.211) (width 0.2) (layer "F.Cu") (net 39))
 (segment (start 106.428 97.072) (end 137.798 97.072) (width 0.2) (layer "F.Cu") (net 39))
 (segment (start 137.798 97.072) (end 139.35 95.52) (width 0.2) (layer "F.Cu") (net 39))
 (segment (start 104.289 99.211) (end 106.428 97.072) (width 0.2) (layer "F.Cu") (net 39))
 (segment (start 102.041 99.211) (end 104.289 99.211) (width 0.2) (layer "F.Cu") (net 39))
 (segment (start 140.501 79.129) (end 140.501 63.651) (width 0.2) (layer "F.Cu") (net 2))
 (segment (start 98.35 62.5) (end 97.199 63.651) (width 0.2) (layer "F.Cu") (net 2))
 (segment (start 105.051 91.591) (end 108.96 95.5) (width 0.2) (layer "F.Cu") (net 2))
 (segment (start 116.5 93) (end 116.5 92.45) (width 0.2) (layer "F.Cu") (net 2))
 (segment (start 101.36676 91.591) (end 105.051 91.591) (width 0.2) (layer "F.Cu") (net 2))
 (segment (start 98.35 62.5) (end 99.501 63.651) (width 0.2) (layer "F.Cu") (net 2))
 (segment (start 140.501 81.431) (end 139.35 80.28) (width 0.2) (layer "F.Cu") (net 2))
 (segment (start 116.5 92.45) (end 118.438 90.512) (width 0.2) (layer "F.Cu") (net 2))
 (segment (start 108.96 95.5) (end 111.46 93) (width 0.2) (layer "F.Cu") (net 2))
 (segment (start 135.47676 92.651) (end 139.07676 89.051) (width 0.2) (layer "F.Cu") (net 2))
 (segment (start 139.07676 89.051) (end 139.82676 89.051) (width 0.2) (layer "F.Cu") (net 2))
 (segment (start 99.501 63.651) (end 108.699838 63.651) (width 0.2) (layer "F.Cu") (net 2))
 (segment (start 108.699838 63.651) (end 109.549838 64.501) (width 0.2) (layer "F.Cu") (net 2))
 (segment (start 140.501 63.651) (end 139.35 62.5) (width 0.2) (layer "F.Cu") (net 2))
 (segment (start 97.199 81.431) (end 97.199 88.37676) (width 0.2) (layer "F.Cu") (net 2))
 (segment (start 97.199 88.37676) (end 97.87324 89.051) (width 0.2) (layer "F.Cu") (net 2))
 (segment (start 129.84424 90.512) (end 131.98324 92.651) (width 0.2) (layer "F.Cu") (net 2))
 (segment (start 118.438 90.512) (end 129.84424 90.512) (width 0.2) (layer "F.Cu") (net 2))
 (segment (start 109.549838 64.501) (end 137.349 64.501) (width 0.2) (layer "F.Cu") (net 2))
 (segment (start 98.35 80.28) (end 97.199 81.431) (width 0.2) (layer "F.Cu") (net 2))
 (segment (start 111.46 93) (end 116.5 93) (width 0.2) (layer "F.Cu") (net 2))
 (segment (start 139.82676 89.051) (end 140.501 88.37676) (width 0.2) (layer "F.Cu") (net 2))
 (segment (start 98.82676 89.051) (end 101.36676 91.591) (width 0.2) (layer "F.Cu") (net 2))
 (segment (start 97.199 79.129) (end 98.35 80.28) (width 0.2) (layer "F.Cu") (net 2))
 (segment (start 137.349 64.501) (end 139.35 62.5) (width 0.2) (layer "F.Cu") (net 2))
 (segment (start 131.98324 92.651) (end 135.47676 92.651) (width 0.2) (layer "F.Cu") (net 2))
 (segment (start 139.35 80.28) (end 140.501 79.129) (width 0.2) (layer "F.Cu") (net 2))
 (segment (start 140.501 88.37676) (end 140.501 81.431) (width 0.2) (layer "F.Cu") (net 2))
 (segment (start 97.199 63.651) (end 97.199 79.129) (width 0.2) (layer "F.Cu") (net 2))
 (segment (start 97.87324 89.051) (end 98.82676 89.051) (width 0.2) (layer "F.Cu") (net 2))
 (segment (start 98.35 98.06) (end 104.791 104.501) (width 0.2) (layer "F.Cu") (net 40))
 (segment (start 132.909 104.501) (end 139.35 98.06) (width 0.2) (layer "F.Cu") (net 40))
 (segment (start 104.791 104.501) (end 132.909 104.501) (width 0.2) (layer "F.Cu") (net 40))
 (segment (start 98.35 75.2) (end 99.501 74.049) (width 0.2) (layer "F.Cu") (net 32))
 (segment (start 99.501 74.049) (end 105.049 74.049) (width 0.2) (layer "F.Cu") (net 32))
 (segment (start 139.259 75.109) (end 139.35 75.2) (width 0.2) (layer "F.Cu") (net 32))
 (segment (start 106.109 75.109) (end 139.259 75.109) (width 0.2) (layer "F.Cu") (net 32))
 (segment (start 105.049 74.049) (end 106.109 75.109) (width 0.2) (layer "F.Cu") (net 32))
 (segment (start 98.35 82.82) (end 99.501 83.971) (width 0.2) (layer "F.Cu") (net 34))
 (segment (start 105.74124 83.971) (end 106.98324 82.729) (width 0.2) (layer "F.Cu") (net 34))
 (segment (start 139.259 82.729) (end 139.35 82.82) (width 0.2) (layer "F.Cu") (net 34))
 (segment (start 99.501 83.971) (end 105.74124 83.971) (width 0.2) (layer "F.Cu") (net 34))
 (segment (start 106.98324 82.729) (end 139.259 82.729) (width 0.2) (layer "F.Cu") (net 34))
 (segment (start 106.98324 90.111) (end 137.139 90.111) (width 0.2) (layer "F.Cu") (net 36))
 (segment (start 105.92324 89.051) (end 106.98324 90.111) (width 0.2) (layer "F.Cu") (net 36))
 (segment (start 99.501 89.051) (end 105.92324 89.051) (width 0.2) (layer "F.Cu") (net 36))
 (segment (start 137.139 90.111) (end 139.35 87.9) (width 0.2) (layer "F.Cu") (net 36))
 (segment (start 98.35 87.9) (end 99.501 89.051) (width 0.2) (layer "F.Cu") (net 36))
 (segment (start 133.119 96.671) (end 139.35 90.44) (width 0.2) (layer "F.Cu") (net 37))
 (segment (start 98.35 90.44) (end 101.849 93.939) (width 0.2) (layer "F.Cu") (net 37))
 (segment (start 101.849 93.939) (end 101.849 95.99676) (width 0.2) (layer "F.Cu") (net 37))
 (segment (start 101.849 95.99676) (end 102.52324 96.671) (width 0.2) (layer "F.Cu") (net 37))
 (segment (start 102.52324 96.671) (end 133.119 96.671) (width 0.2) (layer "F.Cu") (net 37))
 (segment (start 98.35 100.6) (end 102.652 104.902) (width 0.2) (layer "F.Cu") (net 41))
 (segment (start 102.652 104.902) (end 135.048 104.902) (width 0.2) (layer "F.Cu") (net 41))
 (segment (start 135.048 104.902) (end 139.35 100.6) (width 0.2) (layer "F.Cu") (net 41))
 (segment (start 124.2 95.5) (end 122.5 93.8) (width 0.2) (layer "F.Cu") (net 8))
 (segment (start 122.5 93.8) (end 122.5 93) (width 0.2) (layer "F.Cu") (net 8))
 (segment (start 121.66 95.5) (end 121.66 93.16) (width 0.2) (layer "F.Cu") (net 7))
 (segment (start 121.66 93.16) (end 121.5 93) (width 0.2) (layer "F.Cu") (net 7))
 (segment (start 119.12 95.5) (end 120.5 94.12) (width 0.2) (layer "F.Cu") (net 6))
 (segment (start 120.5 94.12) (end 120.5 93) (width 0.2) (layer "F.Cu") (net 6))
 (segment (start 129.32 93) (end 125.5 93) (width 0.2) (layer "F.Cu") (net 11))
 (segment (start 131.82 95.5) (end 129.32 93) (width 0.2) (layer "F.Cu") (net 11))
 (segment (start 124.601 93.651) (end 124.5 93.55) (width 0.2) (layer "F.Cu") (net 10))
 (segment (start 129.28 95.5) (end 127.431 93.651) (width 0.2) (layer "F.Cu") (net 10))
 (segment (start 127.431 93.651) (end 124.601 93.651) (width 0.2) (layer "F.Cu") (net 10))
 (segment (start 124.5 93.55) (end 124.5 93) (width 0.2) (layer "F.Cu") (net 10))
 (segment (start 125.589 94.349) (end 124.349 94.349) (width 0.2) (layer "F.Cu") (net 9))
 (segment (start 126.74 95.5) (end 125.589 94.349) (width 0.2) (layer "F.Cu") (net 9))
 (segment (start 123.5 93.5) (end 123.5 93) (width 0.2) (layer "F.Cu") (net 9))
 (segment (start 124.349 94.349) (end 123.5 93.5) (width 0.2) (layer "F.Cu") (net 9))
 (segment (start 113.101 93.899) (end 117.151 93.899) (width 0.2) (layer "F.Cu") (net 3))
 (segment (start 117.151 93.899) (end 117.5 93.55) (width 0.2) (layer "F.Cu") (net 3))
 (segment (start 111.5 95.5) (end 113.101 93.899) (width 0.2) (layer "F.Cu") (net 3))
 (segment (start 117.5 93.55) (end 117.5 93) (width 0.2) (layer "F.Cu") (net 3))
 (segment (start 119.5 93.49224) (end 119.5 93) (width 0.2) (layer "F.Cu") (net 5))
 (segment (start 116.58 95.5) (end 117.49224 95.5) (width 0.2) (layer "F.Cu") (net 5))
 (segment (start 117.49224 95.5) (end 119.5 93.49224) (width 0.2) (layer "F.Cu") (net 5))
 (segment (start 115.191 94.349) (end 117.701 94.349) (width 0.2) (layer "F.Cu") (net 4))
 (segment (start 117.701 94.349) (end 118.5 93.55) (width 0.2) (layer "F.Cu") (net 4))
 (segment (start 114.04 95.5) (end 115.191 94.349) (width 0.2) (layer "F.Cu") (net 4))
 (segment (start 118.5 93.55) (end 118.5 93) (width 0.2) (layer "F.Cu") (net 4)))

